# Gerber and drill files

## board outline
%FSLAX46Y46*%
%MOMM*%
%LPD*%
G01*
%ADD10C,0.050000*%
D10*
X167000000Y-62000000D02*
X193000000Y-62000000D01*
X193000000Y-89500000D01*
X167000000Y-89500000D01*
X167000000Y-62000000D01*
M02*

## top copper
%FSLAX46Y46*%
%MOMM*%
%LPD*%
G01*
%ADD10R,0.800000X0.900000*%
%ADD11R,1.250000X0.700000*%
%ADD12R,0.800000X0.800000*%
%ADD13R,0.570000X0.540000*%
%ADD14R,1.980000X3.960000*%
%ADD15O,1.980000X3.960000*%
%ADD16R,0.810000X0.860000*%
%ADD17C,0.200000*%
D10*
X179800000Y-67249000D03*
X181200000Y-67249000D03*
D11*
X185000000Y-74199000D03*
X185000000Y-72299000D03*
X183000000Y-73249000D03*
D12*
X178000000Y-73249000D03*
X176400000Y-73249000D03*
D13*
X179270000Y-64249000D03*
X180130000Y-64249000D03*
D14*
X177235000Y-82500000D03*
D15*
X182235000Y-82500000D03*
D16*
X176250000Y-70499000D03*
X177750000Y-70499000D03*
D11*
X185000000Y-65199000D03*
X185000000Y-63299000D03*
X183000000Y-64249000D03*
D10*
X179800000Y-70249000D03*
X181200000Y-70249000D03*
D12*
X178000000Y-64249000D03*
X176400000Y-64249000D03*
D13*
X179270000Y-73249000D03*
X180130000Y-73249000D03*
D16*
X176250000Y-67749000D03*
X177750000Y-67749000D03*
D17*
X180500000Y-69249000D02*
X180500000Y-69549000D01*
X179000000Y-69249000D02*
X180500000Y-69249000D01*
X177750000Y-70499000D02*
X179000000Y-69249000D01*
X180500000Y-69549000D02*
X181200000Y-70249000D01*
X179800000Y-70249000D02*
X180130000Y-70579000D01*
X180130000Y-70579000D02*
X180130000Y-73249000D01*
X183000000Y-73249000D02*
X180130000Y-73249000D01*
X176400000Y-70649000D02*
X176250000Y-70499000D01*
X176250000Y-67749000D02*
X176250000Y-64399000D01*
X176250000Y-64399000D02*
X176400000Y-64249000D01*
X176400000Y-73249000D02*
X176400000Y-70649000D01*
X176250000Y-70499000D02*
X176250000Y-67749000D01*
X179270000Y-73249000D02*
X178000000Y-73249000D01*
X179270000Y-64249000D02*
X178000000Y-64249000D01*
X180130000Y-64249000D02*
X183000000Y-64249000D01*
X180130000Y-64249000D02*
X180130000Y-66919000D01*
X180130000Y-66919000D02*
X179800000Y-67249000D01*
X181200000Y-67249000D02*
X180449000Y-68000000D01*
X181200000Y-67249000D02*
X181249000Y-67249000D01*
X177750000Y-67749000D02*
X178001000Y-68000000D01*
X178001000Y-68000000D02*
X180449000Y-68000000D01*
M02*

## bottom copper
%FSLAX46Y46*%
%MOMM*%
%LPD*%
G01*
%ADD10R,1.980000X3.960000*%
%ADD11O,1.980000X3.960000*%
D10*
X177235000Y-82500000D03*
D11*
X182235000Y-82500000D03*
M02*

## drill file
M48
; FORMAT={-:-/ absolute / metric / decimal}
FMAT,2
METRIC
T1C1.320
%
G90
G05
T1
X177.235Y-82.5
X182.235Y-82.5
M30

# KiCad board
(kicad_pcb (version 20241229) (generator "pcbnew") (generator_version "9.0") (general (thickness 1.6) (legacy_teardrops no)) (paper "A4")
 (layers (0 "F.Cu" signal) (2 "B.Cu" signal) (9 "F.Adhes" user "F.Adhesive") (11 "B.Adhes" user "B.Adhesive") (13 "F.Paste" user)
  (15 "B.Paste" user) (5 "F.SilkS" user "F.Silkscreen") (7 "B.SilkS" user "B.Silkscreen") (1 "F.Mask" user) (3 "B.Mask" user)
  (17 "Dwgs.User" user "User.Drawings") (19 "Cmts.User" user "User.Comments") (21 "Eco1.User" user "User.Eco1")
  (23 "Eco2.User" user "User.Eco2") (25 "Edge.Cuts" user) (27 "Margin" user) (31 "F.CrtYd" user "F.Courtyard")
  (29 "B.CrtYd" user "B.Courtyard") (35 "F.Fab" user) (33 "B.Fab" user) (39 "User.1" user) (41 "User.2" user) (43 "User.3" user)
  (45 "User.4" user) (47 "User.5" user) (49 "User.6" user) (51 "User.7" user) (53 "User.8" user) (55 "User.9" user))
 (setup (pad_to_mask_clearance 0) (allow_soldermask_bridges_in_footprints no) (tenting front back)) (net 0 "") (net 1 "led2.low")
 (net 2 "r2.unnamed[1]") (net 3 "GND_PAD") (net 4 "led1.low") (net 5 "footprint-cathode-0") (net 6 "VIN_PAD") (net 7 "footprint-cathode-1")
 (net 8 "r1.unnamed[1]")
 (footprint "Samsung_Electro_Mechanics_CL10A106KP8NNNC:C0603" (layer "F.Cu") (at 180.5 67.249)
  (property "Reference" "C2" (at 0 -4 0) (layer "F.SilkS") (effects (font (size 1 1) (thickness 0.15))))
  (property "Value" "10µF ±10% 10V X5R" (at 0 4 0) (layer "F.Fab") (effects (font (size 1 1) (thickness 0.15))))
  (pad "1" smd rect (at -0.7 0) (size 0.8 0.9) (layers "F.Cu" "F.Mask" "F.Paste") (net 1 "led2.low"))
  (pad "2" smd rect (at 0.7 0) (size 0.8 0.9) (layers "F.Cu" "F.Mask" "F.Paste") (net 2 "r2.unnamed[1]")))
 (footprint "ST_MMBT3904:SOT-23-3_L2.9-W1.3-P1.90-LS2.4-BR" (layer "F.Cu") (at 184 73.249)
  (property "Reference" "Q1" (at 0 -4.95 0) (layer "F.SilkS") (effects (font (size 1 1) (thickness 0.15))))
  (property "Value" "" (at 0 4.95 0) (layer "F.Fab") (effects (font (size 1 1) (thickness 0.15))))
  (pad "1" smd rect (at 1 0.95) (size 1.25 0.7) (layers "F.Cu" "F.Mask" "F.Paste") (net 2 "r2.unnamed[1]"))
  (pad "2" smd rect (at 1 -0.95) (size 1.25 0.7) (layers "F.Cu" "F.Mask" "F.Paste") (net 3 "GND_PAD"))
  (pad "3" smd rect (at -1 0) (size 1.25 0.7) (layers "F.Cu" "F.Mask" "F.Paste") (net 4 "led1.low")))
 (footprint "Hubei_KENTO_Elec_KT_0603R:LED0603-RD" (layer "F.Cu") (at 177.2 73.249 180)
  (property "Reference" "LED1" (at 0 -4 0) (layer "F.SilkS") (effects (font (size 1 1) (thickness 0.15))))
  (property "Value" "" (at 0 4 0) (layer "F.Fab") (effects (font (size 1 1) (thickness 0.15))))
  (pad "1" smd rect (at -0.8 0 270) (size 0.8 0.8) (layers "F.Cu" "F.Mask" "F.Paste") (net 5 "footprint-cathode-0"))
  (pad "2" smd rect (at 0.8 0 270) (size 0.8 0.8) (layers "F.Cu" "F.Mask" "F.Paste") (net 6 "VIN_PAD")))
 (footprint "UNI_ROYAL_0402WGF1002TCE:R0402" (layer "F.Cu") (at 179.7 64.249)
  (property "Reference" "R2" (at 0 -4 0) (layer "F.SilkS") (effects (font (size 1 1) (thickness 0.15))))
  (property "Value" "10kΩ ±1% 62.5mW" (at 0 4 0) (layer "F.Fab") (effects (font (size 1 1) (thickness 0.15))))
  (pad "1" smd rect (at -0.43 0) (size 0.57 0.54) (layers "F.Cu" "F.Mask" "F.Paste") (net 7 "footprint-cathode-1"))
  (pad "2" smd rect (at 0.43 0) (size 0.57 0.54) (layers "F.Cu" "F.Mask" "F.Paste") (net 1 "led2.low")))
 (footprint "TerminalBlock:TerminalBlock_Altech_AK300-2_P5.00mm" (layer "F.Cu") (at 177.235 82.5)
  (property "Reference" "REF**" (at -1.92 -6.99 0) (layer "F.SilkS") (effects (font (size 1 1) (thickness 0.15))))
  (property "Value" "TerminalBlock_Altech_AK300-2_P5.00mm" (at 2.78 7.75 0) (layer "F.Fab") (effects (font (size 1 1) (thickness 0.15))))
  (pad "1" thru_hole rect (at 0 0) (size 1.98 3.96) (drill 1.32) (layers "*.Cu" "*.Mask") (remove_unused_layers no) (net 6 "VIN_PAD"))
  (pad "2" thru_hole oval (at 5 0) (size 1.98 3.96) (drill 1.32) (layers "*.Cu" "*.Mask") (remove_unused_layers no) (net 3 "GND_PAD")))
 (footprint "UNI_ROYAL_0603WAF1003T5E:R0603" (layer "F.Cu") (at 177 70.499)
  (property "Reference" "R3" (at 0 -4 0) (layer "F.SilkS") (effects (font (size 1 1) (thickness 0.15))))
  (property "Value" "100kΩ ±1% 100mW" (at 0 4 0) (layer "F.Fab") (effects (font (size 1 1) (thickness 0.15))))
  (pad "1" smd rect (at -0.75 0) (size 0.81 0.86) (layers "F.Cu" "F.Mask" "F.Paste") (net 6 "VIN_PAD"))
  (pad "2" smd rect (at 0.75 0) (size 0.81 0.86) (layers "F.Cu" "F.Mask" "F.Paste") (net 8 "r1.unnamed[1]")))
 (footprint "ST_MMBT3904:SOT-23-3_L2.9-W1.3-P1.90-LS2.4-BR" (layer "F.Cu") (at 184 64.249)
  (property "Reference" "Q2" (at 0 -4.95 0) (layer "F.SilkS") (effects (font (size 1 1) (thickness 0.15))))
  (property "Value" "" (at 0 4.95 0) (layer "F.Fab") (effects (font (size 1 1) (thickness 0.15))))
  (pad "1" smd rect (at 1 0.95) (size 1.25 0.7) (layers "F.Cu" "F.Mask" "F.Paste") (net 8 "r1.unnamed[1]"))
  (pad "2" smd rect (at 1 -0.95) (size 1.25 0.7) (layers "F.Cu" "F.Mask" "F.Paste") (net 3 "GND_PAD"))
  (pad "3" smd rect (at -1 0) (size 1.25 0.7) (layers "F.Cu" "F.Mask" "F.Paste") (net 1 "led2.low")))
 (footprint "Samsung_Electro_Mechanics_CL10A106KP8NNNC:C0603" (layer "F.Cu") (at 180.5 70.249)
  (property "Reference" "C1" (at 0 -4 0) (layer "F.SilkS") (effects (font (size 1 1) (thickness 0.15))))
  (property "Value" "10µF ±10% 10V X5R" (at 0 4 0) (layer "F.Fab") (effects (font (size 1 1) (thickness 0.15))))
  (pad "1" smd rect (at -0.7 0) (size 0.8 0.9) (layers "F.Cu" "F.Mask" "F.Paste") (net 4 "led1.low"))
  (pad "2" smd rect (at 0.7 0) (size 0.8 0.9) (layers "F.Cu" "F.Mask" "F.Paste") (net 8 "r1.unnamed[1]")))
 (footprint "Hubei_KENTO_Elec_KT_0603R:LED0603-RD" (layer "F.Cu") (at 177.2 64.249 180)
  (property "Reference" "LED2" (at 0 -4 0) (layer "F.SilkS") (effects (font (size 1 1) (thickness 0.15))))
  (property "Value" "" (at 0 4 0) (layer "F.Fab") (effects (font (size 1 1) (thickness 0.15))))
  (pad "1" smd rect (at -0.8 0 270) (size 0.8 0.8) (layers "F.Cu" "F.Mask" "F.Paste") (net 7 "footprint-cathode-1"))
  (pad "2" smd rect (at 0.8 0 270) (size 0.8 0.8) (layers "F.Cu" "F.Mask" "F.Paste") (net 6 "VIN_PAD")))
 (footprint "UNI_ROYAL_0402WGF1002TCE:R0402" (layer "F.Cu") (at 179.7 73.249)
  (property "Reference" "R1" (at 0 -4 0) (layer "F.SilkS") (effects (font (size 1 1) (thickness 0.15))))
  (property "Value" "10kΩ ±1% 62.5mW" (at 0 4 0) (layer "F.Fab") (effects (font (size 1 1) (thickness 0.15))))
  (pad "1" smd rect (at -0.43 0) (size 0.57 0.54) (layers "F.Cu" "F.Mask" "F.Paste") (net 5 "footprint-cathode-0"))
  (pad "2" smd rect (at 0.43 0) (size 0.57 0.54) (layers "F.Cu" "F.Mask" "F.Paste") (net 4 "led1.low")))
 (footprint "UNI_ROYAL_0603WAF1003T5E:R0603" (layer "F.Cu") (at 177 67.749)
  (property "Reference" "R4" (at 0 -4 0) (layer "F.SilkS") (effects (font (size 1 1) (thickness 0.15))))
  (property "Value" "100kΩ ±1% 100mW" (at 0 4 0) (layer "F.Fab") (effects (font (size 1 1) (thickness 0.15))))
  (pad "1" smd rect (at -0.75 0) (size 0.81 0.86) (layers "F.Cu" "F.Mask" "F.Paste") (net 6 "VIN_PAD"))
  (pad "2" smd rect (at 0.75 0) (size 0.81 0.86) (layers "F.Cu" "F.Mask" "F.Paste") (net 2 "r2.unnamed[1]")))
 (gr_rect (start 167 62) (end 193 89.5) (stroke (width 0.05) (type default)) (fill no) (layer "Edge.Cuts"))
 (segment (start 180.5 69.249) (end 180.5 69.549) (width 0.2) (layer "F.Cu") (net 8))
 (segment (start 179 69.249) (end 180.5 69.249) (width 0.2) (layer "F.Cu") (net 8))
 (segment (start 177.75 70.499) (end 179 69.249) (width 0.2) (layer "F.Cu") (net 8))
 (segment (start 180.5 69.549) (end 181.2 70.249) (width 0.2) (layer "F.Cu") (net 8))
 (segment (start 179.8 70.249) (end 180.13 70.579) (width 0.2) (layer "F.Cu") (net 4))
 (segment (start 180.13 70.579) (end 180.13 73.249) (width 0.2) (layer "F.Cu") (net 4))
 (segment (start 183 73.249) (end 180.13 73.249) (width 0.2) (layer "F.Cu") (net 4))
 (segment (start 176.4 70.649) (end 176.25 70.499) (width 0.2) (layer "F.Cu") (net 6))
 (segment (start 176.25 67.749) (end 176.25 64.399) (width 0.2) (layer "F.Cu") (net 6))
 (segment (start 176.25 64.399) (end 176.4 64.249) (width 0.2) (layer "F.Cu") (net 6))
 (segment (start 176.4 73.249) (end 176.4 70.649) (width 0.2) (layer "F.Cu") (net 6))
 (segment (start 176.25 70.499) (end 176.25 67.749) (width 0.2) (layer "F.Cu") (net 6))
 (segment (start 179.27 73.249) (end 178 73.249) (width 0.2) (layer "F.Cu") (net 5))
 (segment (start 179.27 64.249) (end 178 64.249) (width 0.2) (layer "F.Cu") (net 7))
 (segment (start 180.13 64.249) (end 183 64.249) (width 0.2) (layer "F.Cu") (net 1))
 (segment (start 180.13 64.249) (end 180.13 66.919) (width 0.2) (layer "F.Cu") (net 1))
 (segment (start 180.13 66.919) (end 179.8 67.249) (width 0.2) (layer "F.Cu") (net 1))
 (segment (start 181.2 67.249) (end 180.449 68) (width 0.2) (layer "F.Cu") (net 2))
 (segment (start 181.2 67.249) (end 181.249 67.249) (width 0.2) (layer "F.Cu") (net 2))
 (segment (start 177.75 67.749) (end 178.001 68) (width 0.2) (layer "F.Cu") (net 2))
 (segment (start 178.001 68) (end 180.449 68) (width 0.2) (layer "F.Cu") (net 2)))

